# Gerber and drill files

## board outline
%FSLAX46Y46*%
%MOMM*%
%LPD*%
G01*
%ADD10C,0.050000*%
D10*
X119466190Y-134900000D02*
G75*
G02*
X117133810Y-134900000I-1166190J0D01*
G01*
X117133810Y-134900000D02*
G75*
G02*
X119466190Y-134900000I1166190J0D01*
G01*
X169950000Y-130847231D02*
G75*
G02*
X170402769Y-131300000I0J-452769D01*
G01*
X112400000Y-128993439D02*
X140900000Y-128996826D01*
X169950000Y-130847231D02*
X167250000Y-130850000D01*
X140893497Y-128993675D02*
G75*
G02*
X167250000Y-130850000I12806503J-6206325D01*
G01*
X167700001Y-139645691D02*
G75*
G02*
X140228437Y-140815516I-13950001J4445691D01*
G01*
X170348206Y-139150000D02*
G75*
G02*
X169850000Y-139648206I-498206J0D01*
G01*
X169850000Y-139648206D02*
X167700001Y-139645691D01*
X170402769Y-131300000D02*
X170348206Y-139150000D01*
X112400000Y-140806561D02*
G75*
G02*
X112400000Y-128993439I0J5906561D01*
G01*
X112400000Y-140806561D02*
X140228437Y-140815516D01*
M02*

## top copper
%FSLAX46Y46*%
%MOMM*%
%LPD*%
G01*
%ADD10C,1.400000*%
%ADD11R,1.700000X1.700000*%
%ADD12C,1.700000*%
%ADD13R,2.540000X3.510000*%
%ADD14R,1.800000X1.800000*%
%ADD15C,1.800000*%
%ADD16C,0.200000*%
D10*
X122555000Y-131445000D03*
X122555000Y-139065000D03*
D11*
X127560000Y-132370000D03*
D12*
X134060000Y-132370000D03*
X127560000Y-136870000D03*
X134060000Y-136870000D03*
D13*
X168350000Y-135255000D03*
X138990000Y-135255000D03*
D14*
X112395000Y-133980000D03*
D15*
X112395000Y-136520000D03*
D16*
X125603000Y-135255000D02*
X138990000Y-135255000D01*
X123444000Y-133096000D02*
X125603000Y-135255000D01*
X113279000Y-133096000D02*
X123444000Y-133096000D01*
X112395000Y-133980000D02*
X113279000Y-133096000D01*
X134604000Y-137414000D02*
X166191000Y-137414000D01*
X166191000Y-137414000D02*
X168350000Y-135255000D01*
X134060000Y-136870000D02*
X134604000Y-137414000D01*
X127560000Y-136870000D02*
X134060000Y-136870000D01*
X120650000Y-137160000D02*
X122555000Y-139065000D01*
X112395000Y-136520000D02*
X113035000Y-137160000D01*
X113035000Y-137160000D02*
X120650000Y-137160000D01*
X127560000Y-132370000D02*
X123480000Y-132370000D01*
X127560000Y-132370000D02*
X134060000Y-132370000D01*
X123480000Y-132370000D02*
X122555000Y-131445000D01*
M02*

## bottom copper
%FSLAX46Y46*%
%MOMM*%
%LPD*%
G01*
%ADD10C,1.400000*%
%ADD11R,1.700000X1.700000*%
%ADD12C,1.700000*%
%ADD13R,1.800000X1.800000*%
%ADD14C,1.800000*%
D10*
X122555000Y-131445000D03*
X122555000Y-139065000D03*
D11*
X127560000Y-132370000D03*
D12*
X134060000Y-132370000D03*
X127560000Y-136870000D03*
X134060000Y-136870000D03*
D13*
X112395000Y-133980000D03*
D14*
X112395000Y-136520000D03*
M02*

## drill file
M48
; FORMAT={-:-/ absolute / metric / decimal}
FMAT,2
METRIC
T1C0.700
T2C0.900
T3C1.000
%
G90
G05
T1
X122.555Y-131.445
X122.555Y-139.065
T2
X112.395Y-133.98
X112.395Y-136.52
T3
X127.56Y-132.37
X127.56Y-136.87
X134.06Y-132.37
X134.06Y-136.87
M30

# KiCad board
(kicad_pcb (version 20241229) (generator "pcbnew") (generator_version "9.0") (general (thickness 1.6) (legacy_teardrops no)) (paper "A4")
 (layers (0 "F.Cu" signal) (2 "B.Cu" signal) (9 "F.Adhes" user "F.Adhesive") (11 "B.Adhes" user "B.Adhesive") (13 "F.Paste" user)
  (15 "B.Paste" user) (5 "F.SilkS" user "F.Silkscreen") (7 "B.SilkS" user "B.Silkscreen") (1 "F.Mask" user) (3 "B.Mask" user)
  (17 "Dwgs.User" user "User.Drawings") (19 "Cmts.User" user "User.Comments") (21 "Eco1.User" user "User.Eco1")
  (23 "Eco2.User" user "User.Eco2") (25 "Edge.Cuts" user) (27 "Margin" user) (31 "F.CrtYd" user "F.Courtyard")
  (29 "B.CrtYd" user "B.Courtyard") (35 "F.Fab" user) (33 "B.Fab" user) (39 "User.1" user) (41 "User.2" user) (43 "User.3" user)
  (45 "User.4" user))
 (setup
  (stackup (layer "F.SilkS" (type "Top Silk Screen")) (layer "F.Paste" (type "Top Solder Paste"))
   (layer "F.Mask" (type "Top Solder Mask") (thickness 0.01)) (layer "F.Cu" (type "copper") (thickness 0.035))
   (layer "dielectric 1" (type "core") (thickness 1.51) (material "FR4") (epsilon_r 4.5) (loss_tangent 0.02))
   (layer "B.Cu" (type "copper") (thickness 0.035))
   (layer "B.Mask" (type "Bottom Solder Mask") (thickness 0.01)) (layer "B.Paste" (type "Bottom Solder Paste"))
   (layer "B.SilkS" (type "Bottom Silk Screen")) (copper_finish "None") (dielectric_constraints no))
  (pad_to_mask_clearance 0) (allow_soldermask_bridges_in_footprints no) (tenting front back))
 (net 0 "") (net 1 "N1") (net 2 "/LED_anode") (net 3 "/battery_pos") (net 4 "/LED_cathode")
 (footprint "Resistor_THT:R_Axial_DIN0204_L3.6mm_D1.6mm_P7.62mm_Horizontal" (layer "F.Cu") (at 122.555 131.445 -90)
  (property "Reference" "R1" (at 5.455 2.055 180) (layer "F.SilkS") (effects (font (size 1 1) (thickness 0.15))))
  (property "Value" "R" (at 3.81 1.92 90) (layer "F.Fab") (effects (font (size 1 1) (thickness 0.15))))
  (pad "1" thru_hole circle (at 0 0 270) (size 1.4 1.4) (drill 0.7) (layers "*.Cu" "*.Mask") (remove_unused_layers no) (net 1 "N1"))
  (pad "2" thru_hole circle (at 7.62 0 270) (size 1.4 1.4) (drill 0.7) (layers "*.Cu" "*.Mask") (remove_unused_layers no)
   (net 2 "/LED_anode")))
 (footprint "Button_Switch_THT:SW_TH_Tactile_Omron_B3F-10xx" (layer "F.Cu") (at 127.56 132.37)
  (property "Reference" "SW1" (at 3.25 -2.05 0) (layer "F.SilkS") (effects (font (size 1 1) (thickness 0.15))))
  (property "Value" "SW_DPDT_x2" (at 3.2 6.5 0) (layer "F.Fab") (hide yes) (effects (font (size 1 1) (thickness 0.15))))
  (pad "1" thru_hole rect (at 0 0) (size 1.7 1.7) (drill 1) (layers "*.Cu" "*.Mask") (remove_unused_layers no) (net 1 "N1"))
  (pad "1" thru_hole circle (at 6.5 0) (size 1.7 1.7) (drill 1) (layers "*.Cu" "*.Mask") (remove_unused_layers no) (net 1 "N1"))
  (pad "2" thru_hole circle (at 0 4.5) (size 1.7 1.7) (drill 1) (layers "*.Cu" "*.Mask") (remove_unused_layers no) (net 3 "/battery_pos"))
  (pad "2" thru_hole circle (at 6.5 4.5) (size 1.7 1.7) (drill 1) (layers "*.Cu" "*.Mask") (remove_unused_layers no) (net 3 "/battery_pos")))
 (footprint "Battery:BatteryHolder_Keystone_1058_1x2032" (layer "F.Cu") (at 153.67 135.255 180)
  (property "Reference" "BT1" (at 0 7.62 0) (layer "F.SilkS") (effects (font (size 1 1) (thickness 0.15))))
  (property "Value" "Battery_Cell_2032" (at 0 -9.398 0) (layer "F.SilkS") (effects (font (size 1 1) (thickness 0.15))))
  (pad "1" smd rect (at -14.68 0 180) (size 2.54 3.51) (layers "F.Cu" "F.Mask" "F.Paste") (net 3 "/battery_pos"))
  (pad "2" smd rect (at 14.68 0 180) (size 2.54 3.51) (layers "F.Cu" "F.Mask" "F.Paste") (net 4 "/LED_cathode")))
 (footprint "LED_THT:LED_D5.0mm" (layer "F.Cu") (at 112.395 133.98 -90)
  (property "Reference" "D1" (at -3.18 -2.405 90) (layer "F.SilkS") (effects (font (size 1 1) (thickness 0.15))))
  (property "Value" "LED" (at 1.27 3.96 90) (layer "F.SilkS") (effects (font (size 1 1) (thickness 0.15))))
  (pad "1" thru_hole rect (at 0 0 270) (size 1.8 1.8) (drill 0.9) (layers "*.Cu" "*.Mask") (remove_unused_layers no) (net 4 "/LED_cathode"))
  (pad "2" thru_hole circle (at 2.54 0 270) (size 1.8 1.8) (drill 0.9) (layers "*.Cu" "*.Mask") (remove_unused_layers no)
   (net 2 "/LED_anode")))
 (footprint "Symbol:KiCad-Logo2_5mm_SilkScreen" (layer "B.Cu") (at 153.5 135.255 180)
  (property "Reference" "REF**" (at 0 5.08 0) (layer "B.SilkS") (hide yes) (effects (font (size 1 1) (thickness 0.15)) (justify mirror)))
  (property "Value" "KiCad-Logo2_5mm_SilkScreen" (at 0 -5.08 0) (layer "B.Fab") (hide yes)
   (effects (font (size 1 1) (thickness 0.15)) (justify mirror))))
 (gr_circle (center 118.3 134.9) (end 118.9 133.9) (stroke (width 0.05) (type default)) (fill no) (layer "Edge.Cuts"))
 (gr_arc (start 169.95 130.847231) (mid 170.270156 130.979844) (end 170.402769 131.3) (stroke (width 0.05) (type default)) (locked yes)
  (layer "Edge.Cuts"))
 (gr_line (start 112.4 128.993439) (end 140.9 128.996826) (stroke (width 0.05) (type default)) (locked yes) (layer "Edge.Cuts"))
 (gr_line (start 169.95 130.847231) (end 167.25 130.85) (stroke (width 0.05) (type default)) (locked yes) (layer "Edge.Cuts"))
 (gr_arc (start 140.893497 128.993675) (mid 154.699841 121.004039) (end 167.25 130.85) (stroke (width 0.05) (type default)) (locked yes)
  (layer "Edge.Cuts"))
 (gr_arc (start 167.700001 139.645691) (mid 154.372906 149.82801) (end 140.228437 140.815516) (stroke (width 0.05) (type default))
  (locked yes) (layer "Edge.Cuts"))
 (gr_arc (start 170.348206 139.15) (mid 170.202285 139.502285) (end 169.85 139.648206) (stroke (width 0.05) (type default)) (locked yes)
  (layer "Edge.Cuts"))
 (gr_line (start 169.85 139.648206) (end 167.700001 139.645691) (stroke (width 0.05) (type default)) (locked yes) (layer "Edge.Cuts"))
 (gr_line (start 170.402769 131.3) (end 170.348206 139.15) (stroke (width 0.05) (type default)) (locked yes) (layer "Edge.Cuts"))
 (gr_arc (start 112.4 140.806561) (mid 106.493439 134.9) (end 112.4 128.993439) (stroke (width 0.05) (type default)) (locked yes)
  (layer "Edge.Cuts"))
 (gr_line (start 112.4 140.806561) (end 140.228437 140.815516) (stroke (width 0.05) (type default)) (locked yes) (layer "Edge.Cuts"))
 (segment (start 125.603 135.255) (end 138.99 135.255) (width 0.2) (layer "F.Cu") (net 4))
 (segment (start 123.444 133.096) (end 125.603 135.255) (width 0.2) (layer "F.Cu") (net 4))
 (segment (start 113.279 133.096) (end 123.444 133.096) (width 0.2) (layer "F.Cu") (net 4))
 (segment (start 112.395 133.98) (end 113.279 133.096) (width 0.2) (layer "F.Cu") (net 4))
 (segment (start 134.604 137.414) (end 166.191 137.414) (width 0.2) (layer "F.Cu") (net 3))
 (segment (start 166.191 137.414) (end 168.35 135.255) (width 0.2) (layer "F.Cu") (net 3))
 (segment (start 134.06 136.87) (end 134.604 137.414) (width 0.2) (layer "F.Cu") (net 3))
 (segment (start 127.56 136.87) (end 134.06 136.87) (width 0.2) (layer "F.Cu") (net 3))
 (segment (start 120.65 137.16) (end 122.555 139.065) (width 0.2) (layer "F.Cu") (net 2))
 (segment (start 112.395 136.52) (end 113.035 137.16) (width 0.2) (layer "F.Cu") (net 2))
 (segment (start 113.035 137.16) (end 120.65 137.16) (width 0.2) (layer "F.Cu") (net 2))
 (segment (start 127.56 132.37) (end 123.48 132.37) (width 0.2) (layer "F.Cu") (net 1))
 (segment (start 127.56 132.37) (end 134.06 132.37) (width 0.2) (layer "F.Cu") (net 1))
 (segment (start 123.48 132.37) (end 122.555 131.445) (width 0.2) (layer "F.Cu") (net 1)))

